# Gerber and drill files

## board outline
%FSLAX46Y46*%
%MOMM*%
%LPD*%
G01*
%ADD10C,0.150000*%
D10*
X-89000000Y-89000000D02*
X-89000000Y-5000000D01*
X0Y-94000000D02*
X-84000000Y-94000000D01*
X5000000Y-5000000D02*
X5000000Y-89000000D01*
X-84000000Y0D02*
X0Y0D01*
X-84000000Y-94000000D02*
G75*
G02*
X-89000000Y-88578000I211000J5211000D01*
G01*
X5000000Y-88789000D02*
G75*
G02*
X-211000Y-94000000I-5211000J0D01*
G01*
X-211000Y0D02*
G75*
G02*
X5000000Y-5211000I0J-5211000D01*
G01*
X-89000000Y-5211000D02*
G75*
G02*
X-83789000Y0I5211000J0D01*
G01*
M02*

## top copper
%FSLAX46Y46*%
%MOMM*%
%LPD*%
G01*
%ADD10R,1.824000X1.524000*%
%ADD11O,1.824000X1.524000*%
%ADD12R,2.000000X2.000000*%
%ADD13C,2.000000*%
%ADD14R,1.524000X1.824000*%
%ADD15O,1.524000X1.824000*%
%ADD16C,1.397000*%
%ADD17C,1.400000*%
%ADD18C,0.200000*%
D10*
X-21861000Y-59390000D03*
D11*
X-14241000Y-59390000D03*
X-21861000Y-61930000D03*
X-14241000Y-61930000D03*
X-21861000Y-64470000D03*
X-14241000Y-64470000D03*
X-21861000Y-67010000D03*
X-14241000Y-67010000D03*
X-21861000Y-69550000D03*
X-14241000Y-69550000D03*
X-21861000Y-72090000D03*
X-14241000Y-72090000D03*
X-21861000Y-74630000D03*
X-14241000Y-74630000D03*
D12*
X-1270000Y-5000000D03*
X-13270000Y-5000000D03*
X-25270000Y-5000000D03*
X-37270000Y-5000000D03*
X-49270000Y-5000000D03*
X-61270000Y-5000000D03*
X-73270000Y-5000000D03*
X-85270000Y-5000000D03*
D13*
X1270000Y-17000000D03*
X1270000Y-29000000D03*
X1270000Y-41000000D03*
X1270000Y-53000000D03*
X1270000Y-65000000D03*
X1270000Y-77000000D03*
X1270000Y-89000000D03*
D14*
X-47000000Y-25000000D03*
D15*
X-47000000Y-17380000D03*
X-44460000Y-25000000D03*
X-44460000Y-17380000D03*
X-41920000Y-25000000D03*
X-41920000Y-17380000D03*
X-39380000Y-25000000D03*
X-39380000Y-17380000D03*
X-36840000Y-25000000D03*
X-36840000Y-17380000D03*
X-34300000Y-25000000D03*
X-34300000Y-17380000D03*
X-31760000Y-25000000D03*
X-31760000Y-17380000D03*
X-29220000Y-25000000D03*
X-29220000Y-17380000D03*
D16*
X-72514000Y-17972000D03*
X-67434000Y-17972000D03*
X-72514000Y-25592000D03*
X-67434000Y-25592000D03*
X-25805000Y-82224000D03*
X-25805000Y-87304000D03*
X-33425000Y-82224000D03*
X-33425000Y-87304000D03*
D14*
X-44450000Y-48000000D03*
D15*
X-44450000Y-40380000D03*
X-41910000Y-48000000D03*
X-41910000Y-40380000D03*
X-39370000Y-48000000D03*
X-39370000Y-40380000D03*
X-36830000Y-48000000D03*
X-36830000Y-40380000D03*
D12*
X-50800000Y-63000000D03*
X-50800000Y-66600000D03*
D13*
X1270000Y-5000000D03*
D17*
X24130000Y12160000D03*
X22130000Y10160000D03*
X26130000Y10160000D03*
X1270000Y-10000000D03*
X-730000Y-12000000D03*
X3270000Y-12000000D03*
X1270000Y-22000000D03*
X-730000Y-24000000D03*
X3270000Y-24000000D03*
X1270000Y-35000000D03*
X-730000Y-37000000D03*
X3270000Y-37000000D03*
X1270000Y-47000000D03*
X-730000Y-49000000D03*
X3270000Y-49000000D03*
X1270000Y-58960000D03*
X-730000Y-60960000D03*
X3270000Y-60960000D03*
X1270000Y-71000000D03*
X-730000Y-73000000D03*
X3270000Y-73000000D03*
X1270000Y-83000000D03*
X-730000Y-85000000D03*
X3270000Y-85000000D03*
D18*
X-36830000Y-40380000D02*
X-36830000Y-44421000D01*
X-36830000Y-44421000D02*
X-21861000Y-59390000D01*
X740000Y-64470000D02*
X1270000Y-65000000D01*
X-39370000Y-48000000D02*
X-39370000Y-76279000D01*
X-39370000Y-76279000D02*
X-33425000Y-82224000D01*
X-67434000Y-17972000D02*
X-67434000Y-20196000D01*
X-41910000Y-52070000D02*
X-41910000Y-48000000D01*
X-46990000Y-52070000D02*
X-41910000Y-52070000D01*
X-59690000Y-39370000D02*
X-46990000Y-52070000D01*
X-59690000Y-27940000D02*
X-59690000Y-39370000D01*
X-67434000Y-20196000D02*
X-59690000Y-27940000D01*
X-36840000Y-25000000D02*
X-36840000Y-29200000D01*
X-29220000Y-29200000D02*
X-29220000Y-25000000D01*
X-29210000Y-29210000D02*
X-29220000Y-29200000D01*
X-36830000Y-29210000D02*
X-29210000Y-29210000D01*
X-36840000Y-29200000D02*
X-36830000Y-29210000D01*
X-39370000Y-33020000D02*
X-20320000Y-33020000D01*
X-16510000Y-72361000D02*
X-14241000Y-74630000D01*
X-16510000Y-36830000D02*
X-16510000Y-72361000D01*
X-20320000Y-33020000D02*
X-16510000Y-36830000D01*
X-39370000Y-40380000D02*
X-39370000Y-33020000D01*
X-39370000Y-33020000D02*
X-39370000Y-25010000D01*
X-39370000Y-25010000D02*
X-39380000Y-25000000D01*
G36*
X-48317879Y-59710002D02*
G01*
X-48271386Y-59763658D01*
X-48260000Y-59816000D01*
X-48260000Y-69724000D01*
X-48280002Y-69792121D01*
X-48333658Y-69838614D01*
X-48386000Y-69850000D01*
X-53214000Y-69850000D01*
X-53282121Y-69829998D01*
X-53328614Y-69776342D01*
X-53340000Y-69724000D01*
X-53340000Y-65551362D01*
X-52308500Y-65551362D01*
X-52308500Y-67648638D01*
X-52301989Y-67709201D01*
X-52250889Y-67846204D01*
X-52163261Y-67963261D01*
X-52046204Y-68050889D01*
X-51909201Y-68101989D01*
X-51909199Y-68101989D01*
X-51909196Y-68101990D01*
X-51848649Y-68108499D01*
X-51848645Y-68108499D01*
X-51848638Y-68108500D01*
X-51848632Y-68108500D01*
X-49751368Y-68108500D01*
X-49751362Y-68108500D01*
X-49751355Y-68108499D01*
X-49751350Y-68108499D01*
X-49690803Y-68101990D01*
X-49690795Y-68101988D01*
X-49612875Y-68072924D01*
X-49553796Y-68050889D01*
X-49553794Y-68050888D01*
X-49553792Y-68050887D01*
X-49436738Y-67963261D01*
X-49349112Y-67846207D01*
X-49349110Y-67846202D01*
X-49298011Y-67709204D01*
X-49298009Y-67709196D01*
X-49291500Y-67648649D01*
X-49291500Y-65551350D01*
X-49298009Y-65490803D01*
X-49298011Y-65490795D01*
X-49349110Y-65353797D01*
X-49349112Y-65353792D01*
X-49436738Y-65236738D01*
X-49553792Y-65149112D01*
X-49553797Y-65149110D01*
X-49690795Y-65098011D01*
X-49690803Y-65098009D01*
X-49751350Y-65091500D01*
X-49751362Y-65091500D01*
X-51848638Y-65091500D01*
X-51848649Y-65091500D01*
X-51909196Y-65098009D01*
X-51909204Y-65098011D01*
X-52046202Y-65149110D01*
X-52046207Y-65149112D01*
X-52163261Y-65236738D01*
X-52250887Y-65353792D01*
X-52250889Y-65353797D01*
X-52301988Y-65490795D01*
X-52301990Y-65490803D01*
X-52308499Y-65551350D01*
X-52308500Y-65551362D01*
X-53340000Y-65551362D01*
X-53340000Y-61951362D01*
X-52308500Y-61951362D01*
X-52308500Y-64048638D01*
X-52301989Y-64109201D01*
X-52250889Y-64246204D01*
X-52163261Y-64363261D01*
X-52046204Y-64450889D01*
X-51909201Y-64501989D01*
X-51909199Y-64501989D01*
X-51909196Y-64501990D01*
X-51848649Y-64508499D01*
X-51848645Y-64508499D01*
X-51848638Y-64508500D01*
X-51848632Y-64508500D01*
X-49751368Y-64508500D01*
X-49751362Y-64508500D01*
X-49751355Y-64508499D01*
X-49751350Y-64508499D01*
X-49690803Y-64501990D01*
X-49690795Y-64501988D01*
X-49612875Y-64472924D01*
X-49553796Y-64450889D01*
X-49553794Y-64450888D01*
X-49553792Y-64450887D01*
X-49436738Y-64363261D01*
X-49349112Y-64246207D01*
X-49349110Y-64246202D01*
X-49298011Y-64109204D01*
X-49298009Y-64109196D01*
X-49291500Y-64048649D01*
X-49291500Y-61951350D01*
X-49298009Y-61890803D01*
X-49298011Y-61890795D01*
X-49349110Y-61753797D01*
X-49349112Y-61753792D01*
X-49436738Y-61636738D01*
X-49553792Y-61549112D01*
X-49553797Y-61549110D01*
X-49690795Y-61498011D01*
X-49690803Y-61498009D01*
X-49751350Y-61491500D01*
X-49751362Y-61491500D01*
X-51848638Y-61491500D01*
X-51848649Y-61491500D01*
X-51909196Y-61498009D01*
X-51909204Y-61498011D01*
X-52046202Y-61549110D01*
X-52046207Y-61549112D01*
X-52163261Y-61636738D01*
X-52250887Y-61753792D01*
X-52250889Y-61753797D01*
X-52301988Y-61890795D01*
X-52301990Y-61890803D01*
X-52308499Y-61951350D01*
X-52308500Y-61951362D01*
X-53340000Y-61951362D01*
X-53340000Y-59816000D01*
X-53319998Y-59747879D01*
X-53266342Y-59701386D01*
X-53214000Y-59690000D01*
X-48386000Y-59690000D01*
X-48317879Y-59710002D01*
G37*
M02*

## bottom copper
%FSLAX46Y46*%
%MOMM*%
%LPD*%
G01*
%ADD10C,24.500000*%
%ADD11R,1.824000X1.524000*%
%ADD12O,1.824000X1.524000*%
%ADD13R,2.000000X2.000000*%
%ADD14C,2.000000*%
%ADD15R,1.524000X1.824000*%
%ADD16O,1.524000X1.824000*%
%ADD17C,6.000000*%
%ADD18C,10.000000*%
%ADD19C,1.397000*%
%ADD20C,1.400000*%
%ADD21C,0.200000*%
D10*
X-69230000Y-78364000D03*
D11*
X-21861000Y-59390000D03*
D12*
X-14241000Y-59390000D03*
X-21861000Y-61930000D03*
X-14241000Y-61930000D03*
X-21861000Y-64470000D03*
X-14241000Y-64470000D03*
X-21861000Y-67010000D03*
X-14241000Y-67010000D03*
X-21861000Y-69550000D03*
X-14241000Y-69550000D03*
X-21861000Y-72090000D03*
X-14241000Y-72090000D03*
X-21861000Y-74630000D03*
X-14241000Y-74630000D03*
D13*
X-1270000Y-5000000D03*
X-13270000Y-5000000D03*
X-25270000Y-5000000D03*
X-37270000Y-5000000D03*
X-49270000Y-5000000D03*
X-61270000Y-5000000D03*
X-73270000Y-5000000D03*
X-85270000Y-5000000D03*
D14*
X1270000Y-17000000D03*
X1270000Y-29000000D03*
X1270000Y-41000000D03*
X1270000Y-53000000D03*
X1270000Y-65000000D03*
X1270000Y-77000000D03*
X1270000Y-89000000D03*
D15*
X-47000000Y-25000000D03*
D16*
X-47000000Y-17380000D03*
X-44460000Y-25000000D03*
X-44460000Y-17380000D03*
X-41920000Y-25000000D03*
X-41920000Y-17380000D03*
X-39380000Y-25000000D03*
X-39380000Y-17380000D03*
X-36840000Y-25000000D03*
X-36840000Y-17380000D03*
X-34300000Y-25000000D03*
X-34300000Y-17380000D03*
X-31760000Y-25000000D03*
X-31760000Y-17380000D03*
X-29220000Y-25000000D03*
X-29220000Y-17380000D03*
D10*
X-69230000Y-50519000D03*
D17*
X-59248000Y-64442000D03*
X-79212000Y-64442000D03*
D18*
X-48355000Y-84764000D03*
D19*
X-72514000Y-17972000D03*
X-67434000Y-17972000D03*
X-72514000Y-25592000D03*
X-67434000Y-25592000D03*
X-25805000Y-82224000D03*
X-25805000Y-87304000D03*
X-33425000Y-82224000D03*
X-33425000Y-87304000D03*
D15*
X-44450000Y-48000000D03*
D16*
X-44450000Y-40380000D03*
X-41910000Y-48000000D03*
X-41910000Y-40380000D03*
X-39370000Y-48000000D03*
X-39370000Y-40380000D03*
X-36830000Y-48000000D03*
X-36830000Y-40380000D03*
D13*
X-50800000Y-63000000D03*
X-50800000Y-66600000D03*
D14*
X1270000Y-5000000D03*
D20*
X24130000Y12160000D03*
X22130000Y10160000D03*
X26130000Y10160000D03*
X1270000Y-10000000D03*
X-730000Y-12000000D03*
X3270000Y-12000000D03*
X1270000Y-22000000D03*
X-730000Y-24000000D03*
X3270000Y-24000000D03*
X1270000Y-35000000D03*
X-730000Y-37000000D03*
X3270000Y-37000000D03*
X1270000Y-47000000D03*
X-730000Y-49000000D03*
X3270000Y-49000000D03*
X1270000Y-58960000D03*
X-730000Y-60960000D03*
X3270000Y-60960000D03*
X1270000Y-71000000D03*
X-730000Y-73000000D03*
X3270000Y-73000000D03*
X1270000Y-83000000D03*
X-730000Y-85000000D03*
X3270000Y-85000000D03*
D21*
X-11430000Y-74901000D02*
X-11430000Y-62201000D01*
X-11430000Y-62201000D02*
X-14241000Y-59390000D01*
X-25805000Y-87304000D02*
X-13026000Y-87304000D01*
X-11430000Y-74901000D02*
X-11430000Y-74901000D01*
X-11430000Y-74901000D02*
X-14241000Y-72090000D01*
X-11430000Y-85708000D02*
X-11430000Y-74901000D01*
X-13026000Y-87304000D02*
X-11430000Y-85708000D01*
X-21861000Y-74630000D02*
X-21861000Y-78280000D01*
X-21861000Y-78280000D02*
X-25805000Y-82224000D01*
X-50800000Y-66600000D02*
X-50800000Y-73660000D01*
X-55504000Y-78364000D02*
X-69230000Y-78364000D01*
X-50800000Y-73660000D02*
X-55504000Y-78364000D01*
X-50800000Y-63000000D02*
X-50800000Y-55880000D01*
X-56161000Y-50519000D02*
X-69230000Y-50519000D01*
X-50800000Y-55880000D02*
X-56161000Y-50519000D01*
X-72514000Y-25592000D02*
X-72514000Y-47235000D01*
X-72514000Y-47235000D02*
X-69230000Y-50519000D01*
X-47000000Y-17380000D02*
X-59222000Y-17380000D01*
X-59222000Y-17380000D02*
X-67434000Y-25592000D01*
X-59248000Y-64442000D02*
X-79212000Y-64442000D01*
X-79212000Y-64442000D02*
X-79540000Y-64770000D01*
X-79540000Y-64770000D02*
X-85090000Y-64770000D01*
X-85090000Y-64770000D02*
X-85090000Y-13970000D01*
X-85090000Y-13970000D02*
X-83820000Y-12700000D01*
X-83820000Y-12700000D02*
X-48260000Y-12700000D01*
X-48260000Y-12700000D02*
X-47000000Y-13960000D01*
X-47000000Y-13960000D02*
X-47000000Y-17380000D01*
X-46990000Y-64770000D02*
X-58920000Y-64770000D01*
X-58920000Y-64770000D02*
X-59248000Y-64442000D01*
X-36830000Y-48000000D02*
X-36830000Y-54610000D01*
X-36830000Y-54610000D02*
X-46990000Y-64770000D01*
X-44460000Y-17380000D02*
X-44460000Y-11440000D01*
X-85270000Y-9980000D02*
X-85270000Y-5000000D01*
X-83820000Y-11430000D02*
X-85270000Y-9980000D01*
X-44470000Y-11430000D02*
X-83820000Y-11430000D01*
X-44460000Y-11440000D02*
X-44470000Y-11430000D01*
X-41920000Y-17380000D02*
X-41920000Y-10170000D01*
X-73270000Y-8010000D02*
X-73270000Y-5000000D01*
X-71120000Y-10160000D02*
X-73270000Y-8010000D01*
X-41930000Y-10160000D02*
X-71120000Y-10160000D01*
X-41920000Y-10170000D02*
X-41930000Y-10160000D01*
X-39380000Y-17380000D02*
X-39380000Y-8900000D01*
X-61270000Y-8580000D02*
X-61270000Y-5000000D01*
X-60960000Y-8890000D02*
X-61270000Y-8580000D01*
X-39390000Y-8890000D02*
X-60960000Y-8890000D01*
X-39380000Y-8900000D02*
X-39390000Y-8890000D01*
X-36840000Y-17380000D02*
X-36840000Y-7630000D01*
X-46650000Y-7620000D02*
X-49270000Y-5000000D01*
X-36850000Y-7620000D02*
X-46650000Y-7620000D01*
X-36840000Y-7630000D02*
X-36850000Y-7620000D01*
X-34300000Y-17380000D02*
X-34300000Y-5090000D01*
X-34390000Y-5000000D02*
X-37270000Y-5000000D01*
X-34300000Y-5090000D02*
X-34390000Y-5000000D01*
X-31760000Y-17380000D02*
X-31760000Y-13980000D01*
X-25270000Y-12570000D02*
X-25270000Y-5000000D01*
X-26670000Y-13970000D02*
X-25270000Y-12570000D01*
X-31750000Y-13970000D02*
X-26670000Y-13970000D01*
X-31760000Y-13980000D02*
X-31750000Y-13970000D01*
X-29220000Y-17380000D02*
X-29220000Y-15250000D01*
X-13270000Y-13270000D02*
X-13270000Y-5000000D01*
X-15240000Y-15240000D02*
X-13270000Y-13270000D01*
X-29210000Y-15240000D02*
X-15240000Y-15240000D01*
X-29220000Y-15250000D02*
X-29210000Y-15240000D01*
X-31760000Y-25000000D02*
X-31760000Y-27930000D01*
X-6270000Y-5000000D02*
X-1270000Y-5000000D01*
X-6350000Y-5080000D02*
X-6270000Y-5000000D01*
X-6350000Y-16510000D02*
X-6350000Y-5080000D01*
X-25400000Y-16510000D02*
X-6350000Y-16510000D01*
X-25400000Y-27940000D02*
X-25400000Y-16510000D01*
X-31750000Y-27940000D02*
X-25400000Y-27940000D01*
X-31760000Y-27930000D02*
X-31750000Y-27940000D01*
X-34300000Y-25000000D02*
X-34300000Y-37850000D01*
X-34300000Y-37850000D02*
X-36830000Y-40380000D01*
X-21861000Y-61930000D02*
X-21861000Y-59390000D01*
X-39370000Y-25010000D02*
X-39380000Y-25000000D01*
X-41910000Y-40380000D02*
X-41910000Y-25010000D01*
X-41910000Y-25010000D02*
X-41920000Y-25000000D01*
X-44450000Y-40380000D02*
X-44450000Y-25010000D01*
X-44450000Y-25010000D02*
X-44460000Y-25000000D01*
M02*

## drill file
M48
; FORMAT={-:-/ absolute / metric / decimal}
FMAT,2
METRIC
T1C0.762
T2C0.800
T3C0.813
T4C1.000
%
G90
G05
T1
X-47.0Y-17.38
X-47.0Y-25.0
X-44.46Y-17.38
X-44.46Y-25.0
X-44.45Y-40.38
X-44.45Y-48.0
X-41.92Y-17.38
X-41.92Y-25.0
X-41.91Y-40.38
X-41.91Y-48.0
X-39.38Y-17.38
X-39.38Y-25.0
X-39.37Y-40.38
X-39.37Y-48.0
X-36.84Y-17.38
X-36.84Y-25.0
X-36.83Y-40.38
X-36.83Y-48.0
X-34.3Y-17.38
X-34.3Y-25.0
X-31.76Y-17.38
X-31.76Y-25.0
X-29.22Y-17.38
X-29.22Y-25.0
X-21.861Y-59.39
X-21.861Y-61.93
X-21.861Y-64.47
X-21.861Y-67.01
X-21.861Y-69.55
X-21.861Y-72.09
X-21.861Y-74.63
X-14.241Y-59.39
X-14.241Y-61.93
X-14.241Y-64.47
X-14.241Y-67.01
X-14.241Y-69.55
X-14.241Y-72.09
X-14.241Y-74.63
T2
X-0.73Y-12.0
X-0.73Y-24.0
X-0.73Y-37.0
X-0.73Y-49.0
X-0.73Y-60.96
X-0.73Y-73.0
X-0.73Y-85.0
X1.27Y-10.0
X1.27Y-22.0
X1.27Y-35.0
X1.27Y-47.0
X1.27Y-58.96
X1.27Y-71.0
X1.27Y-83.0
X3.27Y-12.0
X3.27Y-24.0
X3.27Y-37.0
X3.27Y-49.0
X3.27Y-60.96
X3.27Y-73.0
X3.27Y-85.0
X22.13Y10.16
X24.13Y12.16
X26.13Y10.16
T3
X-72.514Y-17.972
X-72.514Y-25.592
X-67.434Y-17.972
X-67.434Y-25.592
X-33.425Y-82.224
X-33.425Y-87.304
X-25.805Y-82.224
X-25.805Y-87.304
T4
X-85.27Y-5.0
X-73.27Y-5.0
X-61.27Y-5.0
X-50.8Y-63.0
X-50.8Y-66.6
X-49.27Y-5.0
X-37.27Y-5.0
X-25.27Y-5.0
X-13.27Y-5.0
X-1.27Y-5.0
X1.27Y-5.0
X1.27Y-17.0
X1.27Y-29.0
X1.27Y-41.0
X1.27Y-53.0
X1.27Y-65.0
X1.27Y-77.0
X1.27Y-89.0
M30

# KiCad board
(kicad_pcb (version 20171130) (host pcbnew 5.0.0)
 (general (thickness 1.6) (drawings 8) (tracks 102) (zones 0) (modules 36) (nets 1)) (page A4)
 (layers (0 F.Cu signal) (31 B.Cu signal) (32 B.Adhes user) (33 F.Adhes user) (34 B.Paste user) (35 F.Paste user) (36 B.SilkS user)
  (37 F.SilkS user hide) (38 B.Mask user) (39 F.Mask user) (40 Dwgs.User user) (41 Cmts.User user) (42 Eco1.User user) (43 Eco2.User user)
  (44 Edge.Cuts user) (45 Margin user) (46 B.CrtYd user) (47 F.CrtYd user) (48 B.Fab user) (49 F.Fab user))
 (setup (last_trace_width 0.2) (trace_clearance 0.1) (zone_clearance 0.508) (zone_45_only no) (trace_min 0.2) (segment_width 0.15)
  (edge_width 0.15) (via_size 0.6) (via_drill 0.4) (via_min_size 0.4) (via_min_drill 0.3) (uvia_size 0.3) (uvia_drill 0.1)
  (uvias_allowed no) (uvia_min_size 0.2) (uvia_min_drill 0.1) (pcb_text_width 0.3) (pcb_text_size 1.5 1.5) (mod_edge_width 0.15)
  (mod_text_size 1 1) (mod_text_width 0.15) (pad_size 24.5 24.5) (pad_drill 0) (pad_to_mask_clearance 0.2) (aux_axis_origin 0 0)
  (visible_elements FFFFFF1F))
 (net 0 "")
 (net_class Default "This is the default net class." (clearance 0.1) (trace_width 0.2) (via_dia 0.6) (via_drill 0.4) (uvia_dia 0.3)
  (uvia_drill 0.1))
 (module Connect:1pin (layer F.Cu) (at -69.23 78.364)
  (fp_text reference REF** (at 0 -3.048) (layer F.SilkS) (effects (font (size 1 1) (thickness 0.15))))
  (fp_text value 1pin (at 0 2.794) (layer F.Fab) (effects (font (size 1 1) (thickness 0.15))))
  (pad 1 smd circle (at 0 0) (size 24.5 24.5) (layers *.Paste *.Mask B.Cu B.SilkS)))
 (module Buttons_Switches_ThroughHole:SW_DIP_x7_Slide (layer F.Cu) (at -21.861 59.39 270)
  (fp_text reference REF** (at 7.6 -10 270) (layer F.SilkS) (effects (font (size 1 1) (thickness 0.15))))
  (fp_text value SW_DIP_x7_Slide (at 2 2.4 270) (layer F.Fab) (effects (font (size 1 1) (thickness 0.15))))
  (pad 1 thru_hole rect (at 0 0 270) (size 1.524 1.824) (drill 0.762) (layers *.Cu *.Mask F.SilkS))
  (pad 14 thru_hole oval (at 0 -7.62 270) (size 1.524 1.824) (drill 0.762) (layers *.Cu *.Adhes *.Paste *.SilkS *.Mask))
  (pad 2 thru_hole oval (at 2.54 0 270) (size 1.524 1.824) (drill 0.762) (layers *.Cu *.Mask F.SilkS))
  (pad 13 thru_hole oval (at 2.54 -7.62 270) (size 1.524 1.824) (drill 0.762) (layers *.Cu *.Mask F.SilkS))
  (pad 3 thru_hole oval (at 5.08 0 270) (size 1.524 1.824) (drill 0.762) (layers *.Cu *.Mask F.SilkS))
  (pad 12 thru_hole oval (at 5.08 -7.62 270) (size 1.524 1.824) (drill 0.762) (layers *.Cu *.Mask F.SilkS))
  (pad 4 thru_hole oval (at 7.62 0 270) (size 1.524 1.824) (drill 0.762) (layers *.Cu *.Mask F.SilkS))
  (pad 11 thru_hole oval (at 7.62 -7.62 270) (size 1.524 1.824) (drill 0.762) (layers *.Cu *.Mask F.SilkS))
  (pad 5 thru_hole oval (at 10.16 0 270) (size 1.524 1.824) (drill 0.762) (layers *.Cu *.Mask F.SilkS))
  (pad 10 thru_hole oval (at 10.16 -7.62 270) (size 1.524 1.824) (drill 0.762) (layers *.Cu *.Mask F.SilkS))
  (pad 6 thru_hole oval (at 12.7 0 270) (size 1.524 1.824) (drill 0.762) (layers *.Cu *.Mask F.SilkS))
  (pad 9 thru_hole oval (at 12.7 -7.62 270) (size 1.524 1.824) (drill 0.762) (layers *.Cu *.Mask F.SilkS))
  (pad 7 thru_hole oval (at 15.24 0 270) (size 1.524 1.824) (drill 0.762) (layers *.Cu *.Mask F.SilkS))
  (pad 8 thru_hole oval (at 15.24 -7.62 270) (size 1.524 1.824) (drill 0.762) (layers *.Cu *.Mask F.SilkS)))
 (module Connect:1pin (layer F.Cu) (at 0 5)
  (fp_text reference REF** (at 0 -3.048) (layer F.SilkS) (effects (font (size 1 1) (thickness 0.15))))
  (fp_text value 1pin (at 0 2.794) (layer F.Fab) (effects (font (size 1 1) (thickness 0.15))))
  (pad 1 thru_hole rect (at -1.27 0) (size 2 2) (drill 1) (layers *.Cu *.Mask F.SilkS)))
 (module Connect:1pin (layer F.Cu) (at -12 5)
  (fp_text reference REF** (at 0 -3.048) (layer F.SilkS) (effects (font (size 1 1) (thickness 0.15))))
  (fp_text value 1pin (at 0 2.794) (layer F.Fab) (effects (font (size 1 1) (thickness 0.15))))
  (pad 1 thru_hole rect (at -1.27 0) (size 2 2) (drill 1) (layers *.Cu *.Mask F.SilkS)))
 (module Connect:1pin (layer F.Cu) (at -24 5)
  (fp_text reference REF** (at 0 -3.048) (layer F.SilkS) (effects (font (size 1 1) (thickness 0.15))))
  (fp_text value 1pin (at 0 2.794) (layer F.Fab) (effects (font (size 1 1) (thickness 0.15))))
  (pad 1 thru_hole rect (at -1.27 0) (size 2 2) (drill 1) (layers *.Cu *.Mask F.SilkS)))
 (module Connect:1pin (layer F.Cu) (at -36 5)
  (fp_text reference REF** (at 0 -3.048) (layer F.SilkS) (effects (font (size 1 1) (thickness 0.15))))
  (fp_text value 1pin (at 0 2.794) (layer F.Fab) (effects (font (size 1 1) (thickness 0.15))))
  (pad 1 thru_hole rect (at -1.27 0) (size 2 2) (drill 1) (layers *.Cu *.Mask F.SilkS)))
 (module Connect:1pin (layer F.Cu) (at -48 5)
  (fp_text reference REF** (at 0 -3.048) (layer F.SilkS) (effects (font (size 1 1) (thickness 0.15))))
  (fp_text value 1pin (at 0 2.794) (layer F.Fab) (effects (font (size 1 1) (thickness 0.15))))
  (pad 1 thru_hole rect (at -1.27 0) (size 2 2) (drill 1) (layers *.Cu *.Mask F.SilkS)))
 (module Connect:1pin (layer F.Cu) (at -60 5)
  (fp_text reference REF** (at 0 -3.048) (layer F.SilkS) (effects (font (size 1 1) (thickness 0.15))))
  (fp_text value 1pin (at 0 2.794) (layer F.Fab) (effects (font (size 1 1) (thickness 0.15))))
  (pad 1 thru_hole rect (at -1.27 0) (size 2 2) (drill 1) (layers *.Cu *.Mask F.SilkS)))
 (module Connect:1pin (layer F.Cu) (at -72 5)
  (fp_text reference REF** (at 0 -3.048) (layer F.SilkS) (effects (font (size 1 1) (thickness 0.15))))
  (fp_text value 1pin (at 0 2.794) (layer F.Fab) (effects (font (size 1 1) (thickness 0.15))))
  (pad 1 thru_hole rect (at -1.27 0) (size 2 2) (drill 1) (layers *.Cu *.Mask F.SilkS)))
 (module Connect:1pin (layer F.Cu) (at -84 5)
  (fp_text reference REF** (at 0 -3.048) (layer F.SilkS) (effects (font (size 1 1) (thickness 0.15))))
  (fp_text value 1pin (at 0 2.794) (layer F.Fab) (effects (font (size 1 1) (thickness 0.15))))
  (pad 1 thru_hole rect (at -1.27 0) (size 2 2) (drill 1) (layers *.Cu *.Mask F.SilkS)))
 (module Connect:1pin (layer F.Cu) (at 0 17)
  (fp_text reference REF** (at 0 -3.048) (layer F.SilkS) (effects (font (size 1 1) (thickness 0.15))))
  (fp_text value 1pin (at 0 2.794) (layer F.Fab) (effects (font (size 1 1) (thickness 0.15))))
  (pad 1 thru_hole circle (at 1.27 0) (size 2 2) (drill 1) (layers *.Cu *.Mask F.SilkS)))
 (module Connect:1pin (layer F.Cu) (at 0 29)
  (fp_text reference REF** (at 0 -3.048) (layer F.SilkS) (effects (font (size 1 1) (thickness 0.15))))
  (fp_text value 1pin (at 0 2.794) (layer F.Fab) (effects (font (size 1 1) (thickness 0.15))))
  (pad 1 thru_hole circle (at 1.27 0) (size 2 2) (drill 1) (layers *.Cu *.Mask F.SilkS)))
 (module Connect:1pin (layer F.Cu) (at 0 41)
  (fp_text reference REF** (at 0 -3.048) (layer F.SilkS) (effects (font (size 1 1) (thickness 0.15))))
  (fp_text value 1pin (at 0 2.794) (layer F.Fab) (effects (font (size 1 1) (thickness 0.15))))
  (pad 1 thru_hole circle (at 1.27 0) (size 2 2) (drill 1) (layers *.Cu *.Mask F.SilkS)))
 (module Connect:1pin (layer F.Cu) (at 0 53)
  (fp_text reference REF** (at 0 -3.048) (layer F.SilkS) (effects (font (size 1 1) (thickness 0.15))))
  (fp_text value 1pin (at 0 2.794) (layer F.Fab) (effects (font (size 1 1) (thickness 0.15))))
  (pad 1 thru_hole circle (at 1.27 0) (size 2 2) (drill 1) (layers *.Cu *.Mask F.SilkS)))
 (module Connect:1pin (layer F.Cu) (at 0 65)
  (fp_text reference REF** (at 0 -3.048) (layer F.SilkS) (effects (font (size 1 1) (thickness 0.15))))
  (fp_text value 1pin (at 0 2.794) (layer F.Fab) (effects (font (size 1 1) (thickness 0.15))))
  (pad 1 thru_hole circle (at 1.27 0) (size 2 2) (drill 1) (layers *.Cu *.Mask F.SilkS)))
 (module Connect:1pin (layer F.Cu) (at 0 77)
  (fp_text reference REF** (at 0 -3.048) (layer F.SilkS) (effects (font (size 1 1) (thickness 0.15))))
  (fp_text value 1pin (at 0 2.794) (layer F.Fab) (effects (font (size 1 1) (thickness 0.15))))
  (pad 1 thru_hole circle (at 1.27 0) (size 2 2) (drill 1) (layers *.Cu *.Mask F.SilkS)))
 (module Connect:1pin (layer F.Cu) (at 0 89)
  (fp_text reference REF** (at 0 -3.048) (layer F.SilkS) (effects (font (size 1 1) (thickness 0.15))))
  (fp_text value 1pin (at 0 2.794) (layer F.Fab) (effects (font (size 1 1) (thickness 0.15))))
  (pad 1 thru_hole circle (at 1.27 0) (size 2 2) (drill 1) (layers *.Cu *.Mask F.SilkS)))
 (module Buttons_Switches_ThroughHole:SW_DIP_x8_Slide (layer F.Cu) (at -47 25)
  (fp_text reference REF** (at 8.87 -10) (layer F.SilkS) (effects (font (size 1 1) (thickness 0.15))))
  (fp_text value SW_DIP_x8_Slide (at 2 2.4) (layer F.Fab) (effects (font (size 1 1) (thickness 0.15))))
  (pad 1 thru_hole rect (at 0 0) (size 1.524 1.824) (drill 0.762) (layers *.Cu *.Mask F.SilkS))
  (pad 16 thru_hole oval (at 0 -7.62) (size 1.524 1.824) (drill 0.762) (layers *.Cu *.Mask F.SilkS))
  (pad 2 thru_hole oval (at 2.54 0) (size 1.524 1.824) (drill 0.762) (layers *.Cu *.Mask F.SilkS))
  (pad 15 thru_hole oval (at 2.54 -7.62) (size 1.524 1.824) (drill 0.762) (layers *.Cu *.Mask F.SilkS))
  (pad 3 thru_hole oval (at 5.08 0) (size 1.524 1.824) (drill 0.762) (layers *.Cu *.Mask F.SilkS))
  (pad 14 thru_hole oval (at 5.08 -7.62) (size 1.524 1.824) (drill 0.762) (layers *.Cu *.Mask F.SilkS))
  (pad 4 thru_hole oval (at 7.62 0) (size 1.524 1.824) (drill 0.762) (layers *.Cu *.Mask F.SilkS))
  (pad 13 thru_hole oval (at 7.62 -7.62) (size 1.524 1.824) (drill 0.762) (layers *.Cu *.Mask F.SilkS))
  (pad 5 thru_hole oval (at 10.16 0) (size 1.524 1.824) (drill 0.762) (layers *.Cu *.Mask F.SilkS))
  (pad 12 thru_hole oval (at 10.16 -7.62) (size 1.524 1.824) (drill 0.762) (layers *.Cu *.Mask F.SilkS))
  (pad 6 thru_hole oval (at 12.7 0) (size 1.524 1.824) (drill 0.762) (layers *.Cu *.Mask F.SilkS))
  (pad 11 thru_hole oval (at 12.7 -7.62) (size 1.524 1.824) (drill 0.762) (layers *.Cu *.Mask F.SilkS))
  (pad 7 thru_hole oval (at 15.24 0) (size 1.524 1.824) (drill 0.762) (layers *.Cu *.Mask F.SilkS))
  (pad 10 thru_hole oval (at 15.24 -7.62) (size 1.524 1.824) (drill 0.762) (layers *.Cu *.Mask F.SilkS))
  (pad 8 thru_hole oval (at 17.78 0) (size 1.524 1.824) (drill 0.762) (layers *.Cu *.Mask F.SilkS))
  (pad 9 thru_hole oval (at 17.78 -7.62) (size 1.524 1.824) (drill 0.762) (layers *.Cu *.Mask F.SilkS)))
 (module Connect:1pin (layer F.Cu) (at -69.23 50.519)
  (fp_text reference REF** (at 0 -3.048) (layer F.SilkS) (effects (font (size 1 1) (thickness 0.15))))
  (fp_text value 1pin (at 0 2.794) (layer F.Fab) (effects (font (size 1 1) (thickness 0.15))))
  (pad 1 smd circle (at 0 0) (size 24.5 24.5) (layers *.Paste *.Mask B.Cu B.SilkS)))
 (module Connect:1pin (layer F.Cu) (at -59.248 64.442)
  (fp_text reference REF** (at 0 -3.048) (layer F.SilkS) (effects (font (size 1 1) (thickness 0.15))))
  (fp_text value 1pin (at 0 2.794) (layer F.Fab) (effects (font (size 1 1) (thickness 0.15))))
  (pad 1 smd circle (at 0 0) (size 6 6) (layers *.Paste *.Mask B.Cu B.SilkS)))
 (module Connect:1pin (layer F.Cu) (at -79.212 64.442)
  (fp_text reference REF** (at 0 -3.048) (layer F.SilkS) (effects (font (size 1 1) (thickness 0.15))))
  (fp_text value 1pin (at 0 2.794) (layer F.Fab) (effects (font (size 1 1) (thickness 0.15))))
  (pad 1 smd circle (at 0 0) (size 6 6) (layers *.Paste *.Mask B.Cu B.SilkS)))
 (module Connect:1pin (layer F.Cu) (at -48.355 84.764)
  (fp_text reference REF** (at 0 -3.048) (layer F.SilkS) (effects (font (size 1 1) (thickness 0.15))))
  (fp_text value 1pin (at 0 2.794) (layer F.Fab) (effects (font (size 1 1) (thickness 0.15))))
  (pad 1 smd circle (at 0 0) (size 10 10) (layers *.Paste *.Mask B.Cu B.SilkS)))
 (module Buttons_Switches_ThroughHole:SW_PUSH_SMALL (layer F.Cu) (at -69.974 21.782 90)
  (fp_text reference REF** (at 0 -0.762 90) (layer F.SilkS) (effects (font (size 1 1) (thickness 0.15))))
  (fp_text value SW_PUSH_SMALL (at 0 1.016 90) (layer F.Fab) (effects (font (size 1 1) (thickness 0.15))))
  (pad 1 thru_hole circle (at 3.81 -2.54 90) (size 1.397 1.397) (drill 0.8128) (layers *.Cu *.Mask F.SilkS))
  (pad 2 thru_hole circle (at 3.81 2.54 90) (size 1.397 1.397) (drill 0.8128) (layers *.Cu *.Mask F.SilkS))
  (pad 1 thru_hole circle (at -3.81 -2.54 90) (size 1.397 1.397) (drill 0.8128) (layers *.Cu *.Mask F.SilkS))
  (pad 2 thru_hole circle (at -3.81 2.54 90) (size 1.397 1.397) (drill 0.8128) (layers *.Cu *.Mask F.SilkS)))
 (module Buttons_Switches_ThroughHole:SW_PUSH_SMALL (layer F.Cu) (at -29.615 84.764)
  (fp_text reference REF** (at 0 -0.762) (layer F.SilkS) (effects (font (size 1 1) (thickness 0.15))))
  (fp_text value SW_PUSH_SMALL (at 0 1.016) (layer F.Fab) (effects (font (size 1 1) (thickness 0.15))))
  (pad 1 thru_hole circle (at 3.81 -2.54) (size 1.397 1.397) (drill 0.8128) (layers *.Cu *.Mask F.SilkS))
  (pad 2 thru_hole circle (at 3.81 2.54) (size 1.397 1.397) (drill 0.8128) (layers *.Cu *.Mask F.SilkS))
  (pad 1 thru_hole circle (at -3.81 -2.54) (size 1.397 1.397) (drill 0.8128) (layers *.Cu *.Mask F.SilkS))
  (pad 2 thru_hole circle (at -3.81 2.54) (size 1.397 1.397) (drill 0.8128) (layers *.Cu *.Mask F.SilkS)))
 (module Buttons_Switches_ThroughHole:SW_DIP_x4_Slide (layer F.Cu) (at -44.45 48)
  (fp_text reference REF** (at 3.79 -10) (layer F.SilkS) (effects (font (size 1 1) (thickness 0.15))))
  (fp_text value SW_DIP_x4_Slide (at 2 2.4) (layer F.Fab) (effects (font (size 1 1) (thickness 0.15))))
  (pad 1 thru_hole rect (at 0 0) (size 1.524 1.824) (drill 0.762) (layers *.Cu *.Mask F.SilkS))
  (pad 8 thru_hole oval (at 0 -7.62) (size 1.524 1.824) (drill 0.762) (layers *.Cu *.Mask F.SilkS))
  (pad 2 thru_hole oval (at 2.54 0) (size 1.524 1.824) (drill 0.762) (layers *.Cu *.Mask F.SilkS))
  (pad 7 thru_hole oval (at 2.54 -7.62) (size 1.524 1.824) (drill 0.762) (layers *.Cu *.Mask F.SilkS))
  (pad 3 thru_hole oval (at 5.08 0) (size 1.524 1.824) (drill 0.762) (layers *.Cu *.Mask F.SilkS))
  (pad 6 thru_hole oval (at 5.08 -7.62) (size 1.524 1.824) (drill 0.762) (layers *.Cu *.Mask F.SilkS))
  (pad 4 thru_hole oval (at 7.62 0) (size 1.524 1.824) (drill 0.762) (layers *.Cu *.Mask F.SilkS))
  (pad 5 thru_hole oval (at 7.62 -7.62) (size 1.524 1.824) (drill 0.762) (layers *.Cu *.Mask F.SilkS)))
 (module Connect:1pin (layer F.Cu) (at -51.27 62.23)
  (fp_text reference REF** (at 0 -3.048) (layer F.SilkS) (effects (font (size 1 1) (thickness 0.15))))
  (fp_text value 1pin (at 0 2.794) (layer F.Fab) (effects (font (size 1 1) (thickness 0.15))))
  (pad 1 thru_hole rect (at 0.47 0.77) (size 2 2) (drill 1) (layers *.Cu *.Mask F.SilkS)))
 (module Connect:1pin (layer F.Cu) (at -50 67.31)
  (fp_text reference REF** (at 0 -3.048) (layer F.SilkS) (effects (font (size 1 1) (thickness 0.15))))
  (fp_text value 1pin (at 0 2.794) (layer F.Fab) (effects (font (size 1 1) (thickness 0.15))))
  (pad 1 thru_hole rect (at -0.8 -0.71) (size 2 2) (drill 1) (layers *.Cu *.Mask F.SilkS)))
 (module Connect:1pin (layer F.Cu) (at 7.62 1.27)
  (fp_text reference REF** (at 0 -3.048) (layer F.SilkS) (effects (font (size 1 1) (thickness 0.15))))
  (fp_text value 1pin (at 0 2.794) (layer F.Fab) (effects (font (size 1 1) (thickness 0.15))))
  (pad 1 thru_hole circle (at -6.35 3.73) (size 2 2) (drill 1) (layers *.Cu *.Mask F.SilkS)))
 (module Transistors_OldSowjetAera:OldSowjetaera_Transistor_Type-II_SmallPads (layer F.Cu) (at 24.13 -10.16)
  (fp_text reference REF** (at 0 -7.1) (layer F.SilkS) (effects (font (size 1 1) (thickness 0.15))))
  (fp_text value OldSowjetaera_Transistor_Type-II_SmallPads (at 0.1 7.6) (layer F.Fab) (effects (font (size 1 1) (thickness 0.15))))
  (pad 2 thru_hole circle (at 0 -2) (size 1.4 1.4) (drill 0.8) (layers *.Cu *.Mask F.SilkS))
  (pad 1 thru_hole circle (at -2 0) (size 1.4 1.4) (drill 0.8) (layers *.Cu *.Mask F.SilkS))
  (pad 3 thru_hole circle (at 2 0) (size 1.4 1.4) (drill 0.8) (layers *.Cu *.Mask F.SilkS)))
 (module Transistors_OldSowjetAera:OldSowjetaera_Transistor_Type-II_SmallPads (layer F.Cu) (at 1.27 12)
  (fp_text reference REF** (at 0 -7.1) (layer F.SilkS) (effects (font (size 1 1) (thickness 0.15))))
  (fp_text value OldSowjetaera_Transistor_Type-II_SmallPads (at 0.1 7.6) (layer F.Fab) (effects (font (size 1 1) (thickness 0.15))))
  (pad 2 thru_hole circle (at 0 -2) (size 1.4 1.4) (drill 0.8) (layers *.Cu *.Mask F.SilkS))
  (pad 1 thru_hole circle (at -2 0) (size 1.4 1.4) (drill 0.8) (layers *.Cu *.Mask F.SilkS))
  (pad 3 thru_hole circle (at 2 0) (size 1.4 1.4) (drill 0.8) (layers *.Cu *.Mask F.SilkS)))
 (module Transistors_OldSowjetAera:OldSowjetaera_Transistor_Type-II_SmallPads (layer F.Cu) (at 1.27 24)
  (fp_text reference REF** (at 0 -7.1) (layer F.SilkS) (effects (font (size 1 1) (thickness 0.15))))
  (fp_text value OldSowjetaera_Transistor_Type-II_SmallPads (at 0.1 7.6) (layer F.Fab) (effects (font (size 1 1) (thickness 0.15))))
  (pad 2 thru_hole circle (at 0 -2) (size 1.4 1.4) (drill 0.8) (layers *.Cu *.Mask F.SilkS))
  (pad 1 thru_hole circle (at -2 0) (size 1.4 1.4) (drill 0.8) (layers *.Cu *.Mask F.SilkS))
  (pad 3 thru_hole circle (at 2 0) (size 1.4 1.4) (drill 0.8) (layers *.Cu *.Mask F.SilkS)))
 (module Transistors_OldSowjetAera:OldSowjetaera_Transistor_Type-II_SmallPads (layer F.Cu) (at 1.27 37)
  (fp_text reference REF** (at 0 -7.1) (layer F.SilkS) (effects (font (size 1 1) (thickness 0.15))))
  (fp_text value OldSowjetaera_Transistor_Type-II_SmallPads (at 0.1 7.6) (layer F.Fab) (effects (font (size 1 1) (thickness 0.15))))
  (pad 2 thru_hole circle (at 0 -2) (size 1.4 1.4) (drill 0.8) (layers *.Cu *.Mask F.SilkS))
  (pad 1 thru_hole circle (at -2 0) (size 1.4 1.4) (drill 0.8) (layers *.Cu *.Mask F.SilkS))
  (pad 3 thru_hole circle (at 2 0) (size 1.4 1.4) (drill 0.8) (layers *.Cu *.Mask F.SilkS)))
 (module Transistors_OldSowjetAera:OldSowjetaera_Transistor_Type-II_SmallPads (layer F.Cu) (at 1.27 49)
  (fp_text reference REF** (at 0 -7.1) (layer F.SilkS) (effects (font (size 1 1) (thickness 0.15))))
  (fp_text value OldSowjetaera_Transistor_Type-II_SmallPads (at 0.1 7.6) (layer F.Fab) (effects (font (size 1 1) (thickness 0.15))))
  (pad 2 thru_hole circle (at 0 -2) (size 1.4 1.4) (drill 0.8) (layers *.Cu *.Mask F.SilkS))
  (pad 1 thru_hole circle (at -2 0) (size 1.4 1.4) (drill 0.8) (layers *.Cu *.Mask F.SilkS))
  (pad 3 thru_hole circle (at 2 0) (size 1.4 1.4) (drill 0.8) (layers *.Cu *.Mask F.SilkS)))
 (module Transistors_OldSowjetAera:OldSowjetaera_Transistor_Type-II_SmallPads (layer F.Cu) (at 1.27 60.96)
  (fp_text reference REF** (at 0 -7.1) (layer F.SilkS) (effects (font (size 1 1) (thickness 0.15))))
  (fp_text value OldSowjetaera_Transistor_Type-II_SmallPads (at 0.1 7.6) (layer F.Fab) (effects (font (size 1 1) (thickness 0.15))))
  (pad 2 thru_hole circle (at 0 -2) (size 1.4 1.4) (drill 0.8) (layers *.Cu *.Mask F.SilkS))
  (pad 1 thru_hole circle (at -2 0) (size 1.4 1.4) (drill 0.8) (layers *.Cu *.Mask F.SilkS))
  (pad 3 thru_hole circle (at 2 0) (size 1.4 1.4) (drill 0.8) (layers *.Cu *.Mask F.SilkS)))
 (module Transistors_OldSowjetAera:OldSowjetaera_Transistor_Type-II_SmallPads (layer F.Cu) (at 1.27 73)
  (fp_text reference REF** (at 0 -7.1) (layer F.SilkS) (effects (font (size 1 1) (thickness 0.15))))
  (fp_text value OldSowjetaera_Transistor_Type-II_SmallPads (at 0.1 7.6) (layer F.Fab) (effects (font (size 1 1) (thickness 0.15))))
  (pad 2 thru_hole circle (at 0 -2) (size 1.4 1.4) (drill 0.8) (layers *.Cu *.Mask F.SilkS))
  (pad 1 thru_hole circle (at -2 0) (size 1.4 1.4) (drill 0.8) (layers *.Cu *.Mask F.SilkS))
  (pad 3 thru_hole circle (at 2 0) (size 1.4 1.4) (drill 0.8) (layers *.Cu *.Mask F.SilkS)))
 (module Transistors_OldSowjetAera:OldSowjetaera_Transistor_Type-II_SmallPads (layer F.Cu) (at 1.27 85)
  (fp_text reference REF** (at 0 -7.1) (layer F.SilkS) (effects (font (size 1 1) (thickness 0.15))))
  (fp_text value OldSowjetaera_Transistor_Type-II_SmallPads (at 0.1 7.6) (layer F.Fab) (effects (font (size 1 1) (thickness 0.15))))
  (pad 2 thru_hole circle (at 0 -2) (size 1.4 1.4) (drill 0.8) (layers *.Cu *.Mask F.SilkS))
  (pad 1 thru_hole circle (at -2 0) (size 1.4 1.4) (drill 0.8) (layers *.Cu *.Mask F.SilkS))
  (pad 3 thru_hole circle (at 2 0) (size 1.4 1.4) (drill 0.8) (layers *.Cu *.Mask F.SilkS)))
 (gr_line (start -89 89) (end -89 5) (angle 90) (layer Edge.Cuts) (width 0.15))
 (gr_line (start 0 94) (end -84 94) (angle 90) (layer Edge.Cuts) (width 0.15))
 (gr_line (start 5 5) (end 5 89) (angle 90) (layer Edge.Cuts) (width 0.15))
 (gr_line (start -84 0) (end 0 0) (angle 90) (layer Edge.Cuts) (width 0.15))
 (gr_arc (start -83.789 88.789) (end -84 94) (angle 90) (layer Edge.Cuts) (width 0.15))
 (gr_arc (start -0.211 88.789) (end 5 88.789) (angle 90) (layer Edge.Cuts) (width 0.15))
 (gr_arc (start -0.211 5.211) (end -0.211 0) (angle 90) (layer Edge.Cuts) (width 0.15))
 (gr_arc (start -83.789 5.211) (end -89 5.211) (angle 90) (layer Edge.Cuts) (width 0.15))
 (segment (start -36.83 40.38) (end -36.83 44.421) (width 0.2) (layer F.Cu) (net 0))
 (segment (start -36.83 44.421) (end -21.861 59.39) (width 0.2) (layer F.Cu) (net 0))
 (segment (start 0.74 64.47) (end 1.27 65) (width 0.2) (layer F.Cu) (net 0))
 (segment (start -11.43 74.901) (end -11.43 62.201) (width 0.2) (layer B.Cu) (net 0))
 (segment (start -11.43 62.201) (end -14.241 59.39) (width 0.2) (layer B.Cu) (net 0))
 (segment (start -25.805 87.304) (end -13.026 87.304) (width 0.2) (layer B.Cu) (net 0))
 (segment (start -11.43 74.901) (end -11.43 74.901) (width 0.2) (layer B.Cu) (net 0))
 (segment (start -11.43 74.901) (end -14.241 72.09) (width 0.2) (layer B.Cu) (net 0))
 (segment (start -11.43 85.708) (end -11.43 74.901) (width 0.2) (layer B.Cu) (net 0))
 (segment (start -13.026 87.304) (end -11.43 85.708) (width 0.2) (layer B.Cu) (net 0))
 (segment (start -21.861 74.63) (end -21.861 78.28) (width 0.2) (layer B.Cu) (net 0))
 (segment (start -21.861 78.28) (end -25.805 82.224) (width 0.2) (layer B.Cu) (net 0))
 (segment (start -39.37 48) (end -39.37 76.279) (width 0.2) (layer F.Cu) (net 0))
 (segment (start -39.37 76.279) (end -33.425 82.224) (width 0.2) (layer F.Cu) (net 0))
 (segment (start -67.434 17.972) (end -67.434 20.196) (width 0.2) (layer F.Cu) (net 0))
 (segment (start -41.91 52.07) (end -41.91 48) (width 0.2) (layer F.Cu) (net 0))
 (segment (start -46.99 52.07) (end -41.91 52.07) (width 0.2) (layer F.Cu) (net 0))
 (segment (start -59.69 39.37) (end -46.99 52.07) (width 0.2) (layer F.Cu) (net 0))
 (segment (start -59.69 27.94) (end -59.69 39.37) (width 0.2) (layer F.Cu) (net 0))
 (segment (start -67.434 20.196) (end -59.69 27.94) (width 0.2) (layer F.Cu) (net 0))
 (segment (start -50.8 66.6) (end -50.8 73.66) (width 0.2) (layer B.Cu) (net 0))
 (segment (start -55.504 78.364) (end -69.23 78.364) (width 0.2) (layer B.Cu) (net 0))
 (segment (start -50.8 73.66) (end -55.504 78.364) (width 0.2) (layer B.Cu) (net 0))
 (segment (start -50.8 63) (end -50.8 55.88) (width 0.2) (layer B.Cu) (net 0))
 (segment (start -56.161 50.519) (end -69.23 50.519) (width 0.2) (layer B.Cu) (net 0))
 (segment (start -50.8 55.88) (end -56.161 50.519) (width 0.2) (layer B.Cu) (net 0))
 (segment (start -72.514 25.592) (end -72.514 47.235) (width 0.2) (layer B.Cu) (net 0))
 (segment (start -72.514 47.235) (end -69.23 50.519) (width 0.2) (layer B.Cu) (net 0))
 (segment (start -47 17.38) (end -59.222 17.38) (width 0.2) (layer B.Cu) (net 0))
 (segment (start -59.222 17.38) (end -67.434 25.592) (width 0.2) (layer B.Cu) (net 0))
 (segment (start -59.248 64.442) (end -79.212 64.442) (width 0.2) (layer B.Cu) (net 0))
 (segment (start -79.212 64.442) (end -79.54 64.77) (width 0.2) (layer B.Cu) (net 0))
 (segment (start -79.54 64.77) (end -85.09 64.77) (width 0.2) (layer B.Cu) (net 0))
 (segment (start -85.09 64.77) (end -85.09 13.97) (width 0.2) (layer B.Cu) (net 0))
 (segment (start -85.09 13.97) (end -83.82 12.7) (width 0.2) (layer B.Cu) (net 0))
 (segment (start -83.82 12.7) (end -48.26 12.7) (width 0.2) (layer B.Cu) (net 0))
 (segment (start -48.26 12.7) (end -47 13.96) (width 0.2) (layer B.Cu) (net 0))
 (segment (start -47 13.96) (end -47 17.38) (width 0.2) (layer B.Cu) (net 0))
 (segment (start -46.99 64.77) (end -58.92 64.77) (width 0.2) (layer B.Cu) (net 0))
 (segment (start -58.92 64.77) (end -59.248 64.442) (width 0.2) (layer B.Cu) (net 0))
 (segment (start -36.83 48) (end -36.83 54.61) (width 0.2) (layer B.Cu) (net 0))
 (segment (start -36.83 54.61) (end -46.99 64.77) (width 0.2) (layer B.Cu) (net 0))
 (segment (start -44.46 17.38) (end -44.46 11.44) (width 0.2) (layer B.Cu) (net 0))
 (segment (start -85.27 9.98) (end -85.27 5) (width 0.2) (layer B.Cu) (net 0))
 (segment (start -83.82 11.43) (end -85.27 9.98) (width 0.2) (layer B.Cu) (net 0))
 (segment (start -44.47 11.43) (end -83.82 11.43) (width 0.2) (layer B.Cu) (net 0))
 (segment (start -44.46 11.44) (end -44.47 11.43) (width 0.2) (layer B.Cu) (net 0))
 (segment (start -41.92 17.38) (end -41.92 10.17) (width 0.2) (layer B.Cu) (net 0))
 (segment (start -73.27 8.01) (end -73.27 5) (width 0.2) (layer B.Cu) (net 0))
 (segment (start -71.12 10.16) (end -73.27 8.01) (width 0.2) (layer B.Cu) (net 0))
 (segment (start -41.93 10.16) (end -71.12 10.16) (width 0.2) (layer B.Cu) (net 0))
 (segment (start -41.92 10.17) (end -41.93 10.16) (width 0.2) (layer B.Cu) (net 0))
 (segment (start -39.38 17.38) (end -39.38 8.9) (width 0.2) (layer B.Cu) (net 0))
 (segment (start -61.27 8.58) (end -61.27 5) (width 0.2) (layer B.Cu) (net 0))
 (segment (start -60.96 8.89) (end -61.27 8.58) (width 0.2) (layer B.Cu) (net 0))
 (segment (start -39.39 8.89) (end -60.96 8.89) (width 0.2) (layer B.Cu) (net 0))
 (segment (start -39.38 8.9) (end -39.39 8.89) (width 0.2) (layer B.Cu) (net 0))
 (segment (start -36.84 17.38) (end -36.84 7.63) (width 0.2) (layer B.Cu) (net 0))
 (segment (start -46.65 7.62) (end -49.27 5) (width 0.2) (layer B.Cu) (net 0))
 (segment (start -36.85 7.62) (end -46.65 7.62) (width 0.2) (layer B.Cu) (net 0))
 (segment (start -36.84 7.63) (end -36.85 7.62) (width 0.2) (layer B.Cu) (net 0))
 (segment (start -34.3 17.38) (end -34.3 5.09) (width 0.2) (layer B.Cu) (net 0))
 (segment (start -34.39 5) (end -37.27 5) (width 0.2) (layer B.Cu) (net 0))
 (segment (start -34.3 5.09) (end -34.39 5) (width 0.2) (layer B.Cu) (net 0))
 (segment (start -31.76 17.38) (end -31.76 13.98) (width 0.2) (layer B.Cu) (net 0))
 (segment (start -25.27 12.57) (end -25.27 5) (width 0.2) (layer B.Cu) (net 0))
 (segment (start -26.67 13.97) (end -25.27 12.57) (width 0.2) (layer B.Cu) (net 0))
 (segment (start -31.75 13.97) (end -26.67 13.97) (width 0.2) (layer B.Cu) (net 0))
 (segment (start -31.76 13.98) (end -31.75 13.97) (width 0.2) (layer B.Cu) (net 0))
 (segment (start -29.22 17.38) (end -29.22 15.25) (width 0.2) (layer B.Cu) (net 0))
 (segment (start -13.27 13.27) (end -13.27 5) (width 0.2) (layer B.Cu) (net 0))
 (segment (start -15.24 15.24) (end -13.27 13.27) (width 0.2) (layer B.Cu) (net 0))
 (segment (start -29.21 15.24) (end -15.24 15.24) (width 0.2) (layer B.Cu) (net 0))
 (segment (start -29.22 15.25) (end -29.21 15.24) (width 0.2) (layer B.Cu) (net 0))
 (segment (start -31.76 25) (end -31.76 27.93) (width 0.2) (layer B.Cu) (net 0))
 (segment (start -6.27 5) (end -1.27 5) (width 0.2) (layer B.Cu) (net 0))
 (segment (start -6.35 5.08) (end -6.27 5) (width 0.2) (layer B.Cu) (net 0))
 (segment (start -6.35 16.51) (end -6.35 5.08) (width 0.2) (layer B.Cu) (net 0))
 (segment (start -25.4 16.51) (end -6.35 16.51) (width 0.2) (layer B.Cu) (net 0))
 (segment (start -25.4 27.94) (end -25.4 16.51) (width 0.2) (layer B.Cu) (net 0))
 (segment (start -31.75 27.94) (end -25.4 27.94) (width 0.2) (layer B.Cu) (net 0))
 (segment (start -31.76 27.93) (end -31.75 27.94) (width 0.2) (layer B.Cu) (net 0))
 (segment (start -36.84 25) (end -36.84 29.2) (width 0.2) (layer F.Cu) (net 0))
 (segment (start -29.22 29.2) (end -29.22 25) (width 0.2) (layer F.Cu) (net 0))
 (segment (start -29.21 29.21) (end -29.22 29.2) (width 0.2) (layer F.Cu) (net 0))
 (segment (start -36.83 29.21) (end -29.21 29.21) (width 0.2) (layer F.Cu) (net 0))
 (segment (start -36.84 29.2) (end -36.83 29.21) (width 0.2) (layer F.Cu) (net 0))
 (segment (start -39.37 33.02) (end -20.32 33.02) (width 0.2) (layer F.Cu) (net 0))
 (segment (start -16.51 72.361) (end -14.241 74.63) (width 0.2) (layer F.Cu) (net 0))
 (segment (start -16.51 36.83) (end -16.51 72.361) (width 0.2) (layer F.Cu) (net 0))
 (segment (start -20.32 33.02) (end -16.51 36.83) (width 0.2) (layer F.Cu) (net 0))
 (segment (start -39.37 40.38) (end -39.37 33.02) (width 0.2) (layer F.Cu) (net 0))
 (segment (start -39.37 33.02) (end -39.37 25.01) (width 0.2) (layer F.Cu) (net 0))
 (segment (start -39.37 25.01) (end -39.38 25) (width 0.2) (layer F.Cu) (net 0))
 (segment (start -34.3 25) (end -34.3 37.85) (width 0.2) (layer B.Cu) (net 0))
 (segment (start -34.3 37.85) (end -36.83 40.38) (width 0.2) (layer B.Cu) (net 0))
 (segment (start -21.861 61.93) (end -21.861 59.39) (width 0.2) (layer B.Cu) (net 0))
 (segment (start -39.37 25.01) (end -39.38 25) (width 0.2) (layer B.Cu) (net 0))
 (segment (start -41.91 40.38) (end -41.91 25.01) (width 0.2) (layer B.Cu) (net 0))
 (segment (start -41.91 25.01) (end -41.92 25) (width 0.2) (layer B.Cu) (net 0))
 (segment (start -44.45 40.38) (end -44.45 25.01) (width 0.2) (layer B.Cu) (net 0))
 (segment (start -44.45 25.01) (end -44.46 25) (width 0.2) (layer B.Cu) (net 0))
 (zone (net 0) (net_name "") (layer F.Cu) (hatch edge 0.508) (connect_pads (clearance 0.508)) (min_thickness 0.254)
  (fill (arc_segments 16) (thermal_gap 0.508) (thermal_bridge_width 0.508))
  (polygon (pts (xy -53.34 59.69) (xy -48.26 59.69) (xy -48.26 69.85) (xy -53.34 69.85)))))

